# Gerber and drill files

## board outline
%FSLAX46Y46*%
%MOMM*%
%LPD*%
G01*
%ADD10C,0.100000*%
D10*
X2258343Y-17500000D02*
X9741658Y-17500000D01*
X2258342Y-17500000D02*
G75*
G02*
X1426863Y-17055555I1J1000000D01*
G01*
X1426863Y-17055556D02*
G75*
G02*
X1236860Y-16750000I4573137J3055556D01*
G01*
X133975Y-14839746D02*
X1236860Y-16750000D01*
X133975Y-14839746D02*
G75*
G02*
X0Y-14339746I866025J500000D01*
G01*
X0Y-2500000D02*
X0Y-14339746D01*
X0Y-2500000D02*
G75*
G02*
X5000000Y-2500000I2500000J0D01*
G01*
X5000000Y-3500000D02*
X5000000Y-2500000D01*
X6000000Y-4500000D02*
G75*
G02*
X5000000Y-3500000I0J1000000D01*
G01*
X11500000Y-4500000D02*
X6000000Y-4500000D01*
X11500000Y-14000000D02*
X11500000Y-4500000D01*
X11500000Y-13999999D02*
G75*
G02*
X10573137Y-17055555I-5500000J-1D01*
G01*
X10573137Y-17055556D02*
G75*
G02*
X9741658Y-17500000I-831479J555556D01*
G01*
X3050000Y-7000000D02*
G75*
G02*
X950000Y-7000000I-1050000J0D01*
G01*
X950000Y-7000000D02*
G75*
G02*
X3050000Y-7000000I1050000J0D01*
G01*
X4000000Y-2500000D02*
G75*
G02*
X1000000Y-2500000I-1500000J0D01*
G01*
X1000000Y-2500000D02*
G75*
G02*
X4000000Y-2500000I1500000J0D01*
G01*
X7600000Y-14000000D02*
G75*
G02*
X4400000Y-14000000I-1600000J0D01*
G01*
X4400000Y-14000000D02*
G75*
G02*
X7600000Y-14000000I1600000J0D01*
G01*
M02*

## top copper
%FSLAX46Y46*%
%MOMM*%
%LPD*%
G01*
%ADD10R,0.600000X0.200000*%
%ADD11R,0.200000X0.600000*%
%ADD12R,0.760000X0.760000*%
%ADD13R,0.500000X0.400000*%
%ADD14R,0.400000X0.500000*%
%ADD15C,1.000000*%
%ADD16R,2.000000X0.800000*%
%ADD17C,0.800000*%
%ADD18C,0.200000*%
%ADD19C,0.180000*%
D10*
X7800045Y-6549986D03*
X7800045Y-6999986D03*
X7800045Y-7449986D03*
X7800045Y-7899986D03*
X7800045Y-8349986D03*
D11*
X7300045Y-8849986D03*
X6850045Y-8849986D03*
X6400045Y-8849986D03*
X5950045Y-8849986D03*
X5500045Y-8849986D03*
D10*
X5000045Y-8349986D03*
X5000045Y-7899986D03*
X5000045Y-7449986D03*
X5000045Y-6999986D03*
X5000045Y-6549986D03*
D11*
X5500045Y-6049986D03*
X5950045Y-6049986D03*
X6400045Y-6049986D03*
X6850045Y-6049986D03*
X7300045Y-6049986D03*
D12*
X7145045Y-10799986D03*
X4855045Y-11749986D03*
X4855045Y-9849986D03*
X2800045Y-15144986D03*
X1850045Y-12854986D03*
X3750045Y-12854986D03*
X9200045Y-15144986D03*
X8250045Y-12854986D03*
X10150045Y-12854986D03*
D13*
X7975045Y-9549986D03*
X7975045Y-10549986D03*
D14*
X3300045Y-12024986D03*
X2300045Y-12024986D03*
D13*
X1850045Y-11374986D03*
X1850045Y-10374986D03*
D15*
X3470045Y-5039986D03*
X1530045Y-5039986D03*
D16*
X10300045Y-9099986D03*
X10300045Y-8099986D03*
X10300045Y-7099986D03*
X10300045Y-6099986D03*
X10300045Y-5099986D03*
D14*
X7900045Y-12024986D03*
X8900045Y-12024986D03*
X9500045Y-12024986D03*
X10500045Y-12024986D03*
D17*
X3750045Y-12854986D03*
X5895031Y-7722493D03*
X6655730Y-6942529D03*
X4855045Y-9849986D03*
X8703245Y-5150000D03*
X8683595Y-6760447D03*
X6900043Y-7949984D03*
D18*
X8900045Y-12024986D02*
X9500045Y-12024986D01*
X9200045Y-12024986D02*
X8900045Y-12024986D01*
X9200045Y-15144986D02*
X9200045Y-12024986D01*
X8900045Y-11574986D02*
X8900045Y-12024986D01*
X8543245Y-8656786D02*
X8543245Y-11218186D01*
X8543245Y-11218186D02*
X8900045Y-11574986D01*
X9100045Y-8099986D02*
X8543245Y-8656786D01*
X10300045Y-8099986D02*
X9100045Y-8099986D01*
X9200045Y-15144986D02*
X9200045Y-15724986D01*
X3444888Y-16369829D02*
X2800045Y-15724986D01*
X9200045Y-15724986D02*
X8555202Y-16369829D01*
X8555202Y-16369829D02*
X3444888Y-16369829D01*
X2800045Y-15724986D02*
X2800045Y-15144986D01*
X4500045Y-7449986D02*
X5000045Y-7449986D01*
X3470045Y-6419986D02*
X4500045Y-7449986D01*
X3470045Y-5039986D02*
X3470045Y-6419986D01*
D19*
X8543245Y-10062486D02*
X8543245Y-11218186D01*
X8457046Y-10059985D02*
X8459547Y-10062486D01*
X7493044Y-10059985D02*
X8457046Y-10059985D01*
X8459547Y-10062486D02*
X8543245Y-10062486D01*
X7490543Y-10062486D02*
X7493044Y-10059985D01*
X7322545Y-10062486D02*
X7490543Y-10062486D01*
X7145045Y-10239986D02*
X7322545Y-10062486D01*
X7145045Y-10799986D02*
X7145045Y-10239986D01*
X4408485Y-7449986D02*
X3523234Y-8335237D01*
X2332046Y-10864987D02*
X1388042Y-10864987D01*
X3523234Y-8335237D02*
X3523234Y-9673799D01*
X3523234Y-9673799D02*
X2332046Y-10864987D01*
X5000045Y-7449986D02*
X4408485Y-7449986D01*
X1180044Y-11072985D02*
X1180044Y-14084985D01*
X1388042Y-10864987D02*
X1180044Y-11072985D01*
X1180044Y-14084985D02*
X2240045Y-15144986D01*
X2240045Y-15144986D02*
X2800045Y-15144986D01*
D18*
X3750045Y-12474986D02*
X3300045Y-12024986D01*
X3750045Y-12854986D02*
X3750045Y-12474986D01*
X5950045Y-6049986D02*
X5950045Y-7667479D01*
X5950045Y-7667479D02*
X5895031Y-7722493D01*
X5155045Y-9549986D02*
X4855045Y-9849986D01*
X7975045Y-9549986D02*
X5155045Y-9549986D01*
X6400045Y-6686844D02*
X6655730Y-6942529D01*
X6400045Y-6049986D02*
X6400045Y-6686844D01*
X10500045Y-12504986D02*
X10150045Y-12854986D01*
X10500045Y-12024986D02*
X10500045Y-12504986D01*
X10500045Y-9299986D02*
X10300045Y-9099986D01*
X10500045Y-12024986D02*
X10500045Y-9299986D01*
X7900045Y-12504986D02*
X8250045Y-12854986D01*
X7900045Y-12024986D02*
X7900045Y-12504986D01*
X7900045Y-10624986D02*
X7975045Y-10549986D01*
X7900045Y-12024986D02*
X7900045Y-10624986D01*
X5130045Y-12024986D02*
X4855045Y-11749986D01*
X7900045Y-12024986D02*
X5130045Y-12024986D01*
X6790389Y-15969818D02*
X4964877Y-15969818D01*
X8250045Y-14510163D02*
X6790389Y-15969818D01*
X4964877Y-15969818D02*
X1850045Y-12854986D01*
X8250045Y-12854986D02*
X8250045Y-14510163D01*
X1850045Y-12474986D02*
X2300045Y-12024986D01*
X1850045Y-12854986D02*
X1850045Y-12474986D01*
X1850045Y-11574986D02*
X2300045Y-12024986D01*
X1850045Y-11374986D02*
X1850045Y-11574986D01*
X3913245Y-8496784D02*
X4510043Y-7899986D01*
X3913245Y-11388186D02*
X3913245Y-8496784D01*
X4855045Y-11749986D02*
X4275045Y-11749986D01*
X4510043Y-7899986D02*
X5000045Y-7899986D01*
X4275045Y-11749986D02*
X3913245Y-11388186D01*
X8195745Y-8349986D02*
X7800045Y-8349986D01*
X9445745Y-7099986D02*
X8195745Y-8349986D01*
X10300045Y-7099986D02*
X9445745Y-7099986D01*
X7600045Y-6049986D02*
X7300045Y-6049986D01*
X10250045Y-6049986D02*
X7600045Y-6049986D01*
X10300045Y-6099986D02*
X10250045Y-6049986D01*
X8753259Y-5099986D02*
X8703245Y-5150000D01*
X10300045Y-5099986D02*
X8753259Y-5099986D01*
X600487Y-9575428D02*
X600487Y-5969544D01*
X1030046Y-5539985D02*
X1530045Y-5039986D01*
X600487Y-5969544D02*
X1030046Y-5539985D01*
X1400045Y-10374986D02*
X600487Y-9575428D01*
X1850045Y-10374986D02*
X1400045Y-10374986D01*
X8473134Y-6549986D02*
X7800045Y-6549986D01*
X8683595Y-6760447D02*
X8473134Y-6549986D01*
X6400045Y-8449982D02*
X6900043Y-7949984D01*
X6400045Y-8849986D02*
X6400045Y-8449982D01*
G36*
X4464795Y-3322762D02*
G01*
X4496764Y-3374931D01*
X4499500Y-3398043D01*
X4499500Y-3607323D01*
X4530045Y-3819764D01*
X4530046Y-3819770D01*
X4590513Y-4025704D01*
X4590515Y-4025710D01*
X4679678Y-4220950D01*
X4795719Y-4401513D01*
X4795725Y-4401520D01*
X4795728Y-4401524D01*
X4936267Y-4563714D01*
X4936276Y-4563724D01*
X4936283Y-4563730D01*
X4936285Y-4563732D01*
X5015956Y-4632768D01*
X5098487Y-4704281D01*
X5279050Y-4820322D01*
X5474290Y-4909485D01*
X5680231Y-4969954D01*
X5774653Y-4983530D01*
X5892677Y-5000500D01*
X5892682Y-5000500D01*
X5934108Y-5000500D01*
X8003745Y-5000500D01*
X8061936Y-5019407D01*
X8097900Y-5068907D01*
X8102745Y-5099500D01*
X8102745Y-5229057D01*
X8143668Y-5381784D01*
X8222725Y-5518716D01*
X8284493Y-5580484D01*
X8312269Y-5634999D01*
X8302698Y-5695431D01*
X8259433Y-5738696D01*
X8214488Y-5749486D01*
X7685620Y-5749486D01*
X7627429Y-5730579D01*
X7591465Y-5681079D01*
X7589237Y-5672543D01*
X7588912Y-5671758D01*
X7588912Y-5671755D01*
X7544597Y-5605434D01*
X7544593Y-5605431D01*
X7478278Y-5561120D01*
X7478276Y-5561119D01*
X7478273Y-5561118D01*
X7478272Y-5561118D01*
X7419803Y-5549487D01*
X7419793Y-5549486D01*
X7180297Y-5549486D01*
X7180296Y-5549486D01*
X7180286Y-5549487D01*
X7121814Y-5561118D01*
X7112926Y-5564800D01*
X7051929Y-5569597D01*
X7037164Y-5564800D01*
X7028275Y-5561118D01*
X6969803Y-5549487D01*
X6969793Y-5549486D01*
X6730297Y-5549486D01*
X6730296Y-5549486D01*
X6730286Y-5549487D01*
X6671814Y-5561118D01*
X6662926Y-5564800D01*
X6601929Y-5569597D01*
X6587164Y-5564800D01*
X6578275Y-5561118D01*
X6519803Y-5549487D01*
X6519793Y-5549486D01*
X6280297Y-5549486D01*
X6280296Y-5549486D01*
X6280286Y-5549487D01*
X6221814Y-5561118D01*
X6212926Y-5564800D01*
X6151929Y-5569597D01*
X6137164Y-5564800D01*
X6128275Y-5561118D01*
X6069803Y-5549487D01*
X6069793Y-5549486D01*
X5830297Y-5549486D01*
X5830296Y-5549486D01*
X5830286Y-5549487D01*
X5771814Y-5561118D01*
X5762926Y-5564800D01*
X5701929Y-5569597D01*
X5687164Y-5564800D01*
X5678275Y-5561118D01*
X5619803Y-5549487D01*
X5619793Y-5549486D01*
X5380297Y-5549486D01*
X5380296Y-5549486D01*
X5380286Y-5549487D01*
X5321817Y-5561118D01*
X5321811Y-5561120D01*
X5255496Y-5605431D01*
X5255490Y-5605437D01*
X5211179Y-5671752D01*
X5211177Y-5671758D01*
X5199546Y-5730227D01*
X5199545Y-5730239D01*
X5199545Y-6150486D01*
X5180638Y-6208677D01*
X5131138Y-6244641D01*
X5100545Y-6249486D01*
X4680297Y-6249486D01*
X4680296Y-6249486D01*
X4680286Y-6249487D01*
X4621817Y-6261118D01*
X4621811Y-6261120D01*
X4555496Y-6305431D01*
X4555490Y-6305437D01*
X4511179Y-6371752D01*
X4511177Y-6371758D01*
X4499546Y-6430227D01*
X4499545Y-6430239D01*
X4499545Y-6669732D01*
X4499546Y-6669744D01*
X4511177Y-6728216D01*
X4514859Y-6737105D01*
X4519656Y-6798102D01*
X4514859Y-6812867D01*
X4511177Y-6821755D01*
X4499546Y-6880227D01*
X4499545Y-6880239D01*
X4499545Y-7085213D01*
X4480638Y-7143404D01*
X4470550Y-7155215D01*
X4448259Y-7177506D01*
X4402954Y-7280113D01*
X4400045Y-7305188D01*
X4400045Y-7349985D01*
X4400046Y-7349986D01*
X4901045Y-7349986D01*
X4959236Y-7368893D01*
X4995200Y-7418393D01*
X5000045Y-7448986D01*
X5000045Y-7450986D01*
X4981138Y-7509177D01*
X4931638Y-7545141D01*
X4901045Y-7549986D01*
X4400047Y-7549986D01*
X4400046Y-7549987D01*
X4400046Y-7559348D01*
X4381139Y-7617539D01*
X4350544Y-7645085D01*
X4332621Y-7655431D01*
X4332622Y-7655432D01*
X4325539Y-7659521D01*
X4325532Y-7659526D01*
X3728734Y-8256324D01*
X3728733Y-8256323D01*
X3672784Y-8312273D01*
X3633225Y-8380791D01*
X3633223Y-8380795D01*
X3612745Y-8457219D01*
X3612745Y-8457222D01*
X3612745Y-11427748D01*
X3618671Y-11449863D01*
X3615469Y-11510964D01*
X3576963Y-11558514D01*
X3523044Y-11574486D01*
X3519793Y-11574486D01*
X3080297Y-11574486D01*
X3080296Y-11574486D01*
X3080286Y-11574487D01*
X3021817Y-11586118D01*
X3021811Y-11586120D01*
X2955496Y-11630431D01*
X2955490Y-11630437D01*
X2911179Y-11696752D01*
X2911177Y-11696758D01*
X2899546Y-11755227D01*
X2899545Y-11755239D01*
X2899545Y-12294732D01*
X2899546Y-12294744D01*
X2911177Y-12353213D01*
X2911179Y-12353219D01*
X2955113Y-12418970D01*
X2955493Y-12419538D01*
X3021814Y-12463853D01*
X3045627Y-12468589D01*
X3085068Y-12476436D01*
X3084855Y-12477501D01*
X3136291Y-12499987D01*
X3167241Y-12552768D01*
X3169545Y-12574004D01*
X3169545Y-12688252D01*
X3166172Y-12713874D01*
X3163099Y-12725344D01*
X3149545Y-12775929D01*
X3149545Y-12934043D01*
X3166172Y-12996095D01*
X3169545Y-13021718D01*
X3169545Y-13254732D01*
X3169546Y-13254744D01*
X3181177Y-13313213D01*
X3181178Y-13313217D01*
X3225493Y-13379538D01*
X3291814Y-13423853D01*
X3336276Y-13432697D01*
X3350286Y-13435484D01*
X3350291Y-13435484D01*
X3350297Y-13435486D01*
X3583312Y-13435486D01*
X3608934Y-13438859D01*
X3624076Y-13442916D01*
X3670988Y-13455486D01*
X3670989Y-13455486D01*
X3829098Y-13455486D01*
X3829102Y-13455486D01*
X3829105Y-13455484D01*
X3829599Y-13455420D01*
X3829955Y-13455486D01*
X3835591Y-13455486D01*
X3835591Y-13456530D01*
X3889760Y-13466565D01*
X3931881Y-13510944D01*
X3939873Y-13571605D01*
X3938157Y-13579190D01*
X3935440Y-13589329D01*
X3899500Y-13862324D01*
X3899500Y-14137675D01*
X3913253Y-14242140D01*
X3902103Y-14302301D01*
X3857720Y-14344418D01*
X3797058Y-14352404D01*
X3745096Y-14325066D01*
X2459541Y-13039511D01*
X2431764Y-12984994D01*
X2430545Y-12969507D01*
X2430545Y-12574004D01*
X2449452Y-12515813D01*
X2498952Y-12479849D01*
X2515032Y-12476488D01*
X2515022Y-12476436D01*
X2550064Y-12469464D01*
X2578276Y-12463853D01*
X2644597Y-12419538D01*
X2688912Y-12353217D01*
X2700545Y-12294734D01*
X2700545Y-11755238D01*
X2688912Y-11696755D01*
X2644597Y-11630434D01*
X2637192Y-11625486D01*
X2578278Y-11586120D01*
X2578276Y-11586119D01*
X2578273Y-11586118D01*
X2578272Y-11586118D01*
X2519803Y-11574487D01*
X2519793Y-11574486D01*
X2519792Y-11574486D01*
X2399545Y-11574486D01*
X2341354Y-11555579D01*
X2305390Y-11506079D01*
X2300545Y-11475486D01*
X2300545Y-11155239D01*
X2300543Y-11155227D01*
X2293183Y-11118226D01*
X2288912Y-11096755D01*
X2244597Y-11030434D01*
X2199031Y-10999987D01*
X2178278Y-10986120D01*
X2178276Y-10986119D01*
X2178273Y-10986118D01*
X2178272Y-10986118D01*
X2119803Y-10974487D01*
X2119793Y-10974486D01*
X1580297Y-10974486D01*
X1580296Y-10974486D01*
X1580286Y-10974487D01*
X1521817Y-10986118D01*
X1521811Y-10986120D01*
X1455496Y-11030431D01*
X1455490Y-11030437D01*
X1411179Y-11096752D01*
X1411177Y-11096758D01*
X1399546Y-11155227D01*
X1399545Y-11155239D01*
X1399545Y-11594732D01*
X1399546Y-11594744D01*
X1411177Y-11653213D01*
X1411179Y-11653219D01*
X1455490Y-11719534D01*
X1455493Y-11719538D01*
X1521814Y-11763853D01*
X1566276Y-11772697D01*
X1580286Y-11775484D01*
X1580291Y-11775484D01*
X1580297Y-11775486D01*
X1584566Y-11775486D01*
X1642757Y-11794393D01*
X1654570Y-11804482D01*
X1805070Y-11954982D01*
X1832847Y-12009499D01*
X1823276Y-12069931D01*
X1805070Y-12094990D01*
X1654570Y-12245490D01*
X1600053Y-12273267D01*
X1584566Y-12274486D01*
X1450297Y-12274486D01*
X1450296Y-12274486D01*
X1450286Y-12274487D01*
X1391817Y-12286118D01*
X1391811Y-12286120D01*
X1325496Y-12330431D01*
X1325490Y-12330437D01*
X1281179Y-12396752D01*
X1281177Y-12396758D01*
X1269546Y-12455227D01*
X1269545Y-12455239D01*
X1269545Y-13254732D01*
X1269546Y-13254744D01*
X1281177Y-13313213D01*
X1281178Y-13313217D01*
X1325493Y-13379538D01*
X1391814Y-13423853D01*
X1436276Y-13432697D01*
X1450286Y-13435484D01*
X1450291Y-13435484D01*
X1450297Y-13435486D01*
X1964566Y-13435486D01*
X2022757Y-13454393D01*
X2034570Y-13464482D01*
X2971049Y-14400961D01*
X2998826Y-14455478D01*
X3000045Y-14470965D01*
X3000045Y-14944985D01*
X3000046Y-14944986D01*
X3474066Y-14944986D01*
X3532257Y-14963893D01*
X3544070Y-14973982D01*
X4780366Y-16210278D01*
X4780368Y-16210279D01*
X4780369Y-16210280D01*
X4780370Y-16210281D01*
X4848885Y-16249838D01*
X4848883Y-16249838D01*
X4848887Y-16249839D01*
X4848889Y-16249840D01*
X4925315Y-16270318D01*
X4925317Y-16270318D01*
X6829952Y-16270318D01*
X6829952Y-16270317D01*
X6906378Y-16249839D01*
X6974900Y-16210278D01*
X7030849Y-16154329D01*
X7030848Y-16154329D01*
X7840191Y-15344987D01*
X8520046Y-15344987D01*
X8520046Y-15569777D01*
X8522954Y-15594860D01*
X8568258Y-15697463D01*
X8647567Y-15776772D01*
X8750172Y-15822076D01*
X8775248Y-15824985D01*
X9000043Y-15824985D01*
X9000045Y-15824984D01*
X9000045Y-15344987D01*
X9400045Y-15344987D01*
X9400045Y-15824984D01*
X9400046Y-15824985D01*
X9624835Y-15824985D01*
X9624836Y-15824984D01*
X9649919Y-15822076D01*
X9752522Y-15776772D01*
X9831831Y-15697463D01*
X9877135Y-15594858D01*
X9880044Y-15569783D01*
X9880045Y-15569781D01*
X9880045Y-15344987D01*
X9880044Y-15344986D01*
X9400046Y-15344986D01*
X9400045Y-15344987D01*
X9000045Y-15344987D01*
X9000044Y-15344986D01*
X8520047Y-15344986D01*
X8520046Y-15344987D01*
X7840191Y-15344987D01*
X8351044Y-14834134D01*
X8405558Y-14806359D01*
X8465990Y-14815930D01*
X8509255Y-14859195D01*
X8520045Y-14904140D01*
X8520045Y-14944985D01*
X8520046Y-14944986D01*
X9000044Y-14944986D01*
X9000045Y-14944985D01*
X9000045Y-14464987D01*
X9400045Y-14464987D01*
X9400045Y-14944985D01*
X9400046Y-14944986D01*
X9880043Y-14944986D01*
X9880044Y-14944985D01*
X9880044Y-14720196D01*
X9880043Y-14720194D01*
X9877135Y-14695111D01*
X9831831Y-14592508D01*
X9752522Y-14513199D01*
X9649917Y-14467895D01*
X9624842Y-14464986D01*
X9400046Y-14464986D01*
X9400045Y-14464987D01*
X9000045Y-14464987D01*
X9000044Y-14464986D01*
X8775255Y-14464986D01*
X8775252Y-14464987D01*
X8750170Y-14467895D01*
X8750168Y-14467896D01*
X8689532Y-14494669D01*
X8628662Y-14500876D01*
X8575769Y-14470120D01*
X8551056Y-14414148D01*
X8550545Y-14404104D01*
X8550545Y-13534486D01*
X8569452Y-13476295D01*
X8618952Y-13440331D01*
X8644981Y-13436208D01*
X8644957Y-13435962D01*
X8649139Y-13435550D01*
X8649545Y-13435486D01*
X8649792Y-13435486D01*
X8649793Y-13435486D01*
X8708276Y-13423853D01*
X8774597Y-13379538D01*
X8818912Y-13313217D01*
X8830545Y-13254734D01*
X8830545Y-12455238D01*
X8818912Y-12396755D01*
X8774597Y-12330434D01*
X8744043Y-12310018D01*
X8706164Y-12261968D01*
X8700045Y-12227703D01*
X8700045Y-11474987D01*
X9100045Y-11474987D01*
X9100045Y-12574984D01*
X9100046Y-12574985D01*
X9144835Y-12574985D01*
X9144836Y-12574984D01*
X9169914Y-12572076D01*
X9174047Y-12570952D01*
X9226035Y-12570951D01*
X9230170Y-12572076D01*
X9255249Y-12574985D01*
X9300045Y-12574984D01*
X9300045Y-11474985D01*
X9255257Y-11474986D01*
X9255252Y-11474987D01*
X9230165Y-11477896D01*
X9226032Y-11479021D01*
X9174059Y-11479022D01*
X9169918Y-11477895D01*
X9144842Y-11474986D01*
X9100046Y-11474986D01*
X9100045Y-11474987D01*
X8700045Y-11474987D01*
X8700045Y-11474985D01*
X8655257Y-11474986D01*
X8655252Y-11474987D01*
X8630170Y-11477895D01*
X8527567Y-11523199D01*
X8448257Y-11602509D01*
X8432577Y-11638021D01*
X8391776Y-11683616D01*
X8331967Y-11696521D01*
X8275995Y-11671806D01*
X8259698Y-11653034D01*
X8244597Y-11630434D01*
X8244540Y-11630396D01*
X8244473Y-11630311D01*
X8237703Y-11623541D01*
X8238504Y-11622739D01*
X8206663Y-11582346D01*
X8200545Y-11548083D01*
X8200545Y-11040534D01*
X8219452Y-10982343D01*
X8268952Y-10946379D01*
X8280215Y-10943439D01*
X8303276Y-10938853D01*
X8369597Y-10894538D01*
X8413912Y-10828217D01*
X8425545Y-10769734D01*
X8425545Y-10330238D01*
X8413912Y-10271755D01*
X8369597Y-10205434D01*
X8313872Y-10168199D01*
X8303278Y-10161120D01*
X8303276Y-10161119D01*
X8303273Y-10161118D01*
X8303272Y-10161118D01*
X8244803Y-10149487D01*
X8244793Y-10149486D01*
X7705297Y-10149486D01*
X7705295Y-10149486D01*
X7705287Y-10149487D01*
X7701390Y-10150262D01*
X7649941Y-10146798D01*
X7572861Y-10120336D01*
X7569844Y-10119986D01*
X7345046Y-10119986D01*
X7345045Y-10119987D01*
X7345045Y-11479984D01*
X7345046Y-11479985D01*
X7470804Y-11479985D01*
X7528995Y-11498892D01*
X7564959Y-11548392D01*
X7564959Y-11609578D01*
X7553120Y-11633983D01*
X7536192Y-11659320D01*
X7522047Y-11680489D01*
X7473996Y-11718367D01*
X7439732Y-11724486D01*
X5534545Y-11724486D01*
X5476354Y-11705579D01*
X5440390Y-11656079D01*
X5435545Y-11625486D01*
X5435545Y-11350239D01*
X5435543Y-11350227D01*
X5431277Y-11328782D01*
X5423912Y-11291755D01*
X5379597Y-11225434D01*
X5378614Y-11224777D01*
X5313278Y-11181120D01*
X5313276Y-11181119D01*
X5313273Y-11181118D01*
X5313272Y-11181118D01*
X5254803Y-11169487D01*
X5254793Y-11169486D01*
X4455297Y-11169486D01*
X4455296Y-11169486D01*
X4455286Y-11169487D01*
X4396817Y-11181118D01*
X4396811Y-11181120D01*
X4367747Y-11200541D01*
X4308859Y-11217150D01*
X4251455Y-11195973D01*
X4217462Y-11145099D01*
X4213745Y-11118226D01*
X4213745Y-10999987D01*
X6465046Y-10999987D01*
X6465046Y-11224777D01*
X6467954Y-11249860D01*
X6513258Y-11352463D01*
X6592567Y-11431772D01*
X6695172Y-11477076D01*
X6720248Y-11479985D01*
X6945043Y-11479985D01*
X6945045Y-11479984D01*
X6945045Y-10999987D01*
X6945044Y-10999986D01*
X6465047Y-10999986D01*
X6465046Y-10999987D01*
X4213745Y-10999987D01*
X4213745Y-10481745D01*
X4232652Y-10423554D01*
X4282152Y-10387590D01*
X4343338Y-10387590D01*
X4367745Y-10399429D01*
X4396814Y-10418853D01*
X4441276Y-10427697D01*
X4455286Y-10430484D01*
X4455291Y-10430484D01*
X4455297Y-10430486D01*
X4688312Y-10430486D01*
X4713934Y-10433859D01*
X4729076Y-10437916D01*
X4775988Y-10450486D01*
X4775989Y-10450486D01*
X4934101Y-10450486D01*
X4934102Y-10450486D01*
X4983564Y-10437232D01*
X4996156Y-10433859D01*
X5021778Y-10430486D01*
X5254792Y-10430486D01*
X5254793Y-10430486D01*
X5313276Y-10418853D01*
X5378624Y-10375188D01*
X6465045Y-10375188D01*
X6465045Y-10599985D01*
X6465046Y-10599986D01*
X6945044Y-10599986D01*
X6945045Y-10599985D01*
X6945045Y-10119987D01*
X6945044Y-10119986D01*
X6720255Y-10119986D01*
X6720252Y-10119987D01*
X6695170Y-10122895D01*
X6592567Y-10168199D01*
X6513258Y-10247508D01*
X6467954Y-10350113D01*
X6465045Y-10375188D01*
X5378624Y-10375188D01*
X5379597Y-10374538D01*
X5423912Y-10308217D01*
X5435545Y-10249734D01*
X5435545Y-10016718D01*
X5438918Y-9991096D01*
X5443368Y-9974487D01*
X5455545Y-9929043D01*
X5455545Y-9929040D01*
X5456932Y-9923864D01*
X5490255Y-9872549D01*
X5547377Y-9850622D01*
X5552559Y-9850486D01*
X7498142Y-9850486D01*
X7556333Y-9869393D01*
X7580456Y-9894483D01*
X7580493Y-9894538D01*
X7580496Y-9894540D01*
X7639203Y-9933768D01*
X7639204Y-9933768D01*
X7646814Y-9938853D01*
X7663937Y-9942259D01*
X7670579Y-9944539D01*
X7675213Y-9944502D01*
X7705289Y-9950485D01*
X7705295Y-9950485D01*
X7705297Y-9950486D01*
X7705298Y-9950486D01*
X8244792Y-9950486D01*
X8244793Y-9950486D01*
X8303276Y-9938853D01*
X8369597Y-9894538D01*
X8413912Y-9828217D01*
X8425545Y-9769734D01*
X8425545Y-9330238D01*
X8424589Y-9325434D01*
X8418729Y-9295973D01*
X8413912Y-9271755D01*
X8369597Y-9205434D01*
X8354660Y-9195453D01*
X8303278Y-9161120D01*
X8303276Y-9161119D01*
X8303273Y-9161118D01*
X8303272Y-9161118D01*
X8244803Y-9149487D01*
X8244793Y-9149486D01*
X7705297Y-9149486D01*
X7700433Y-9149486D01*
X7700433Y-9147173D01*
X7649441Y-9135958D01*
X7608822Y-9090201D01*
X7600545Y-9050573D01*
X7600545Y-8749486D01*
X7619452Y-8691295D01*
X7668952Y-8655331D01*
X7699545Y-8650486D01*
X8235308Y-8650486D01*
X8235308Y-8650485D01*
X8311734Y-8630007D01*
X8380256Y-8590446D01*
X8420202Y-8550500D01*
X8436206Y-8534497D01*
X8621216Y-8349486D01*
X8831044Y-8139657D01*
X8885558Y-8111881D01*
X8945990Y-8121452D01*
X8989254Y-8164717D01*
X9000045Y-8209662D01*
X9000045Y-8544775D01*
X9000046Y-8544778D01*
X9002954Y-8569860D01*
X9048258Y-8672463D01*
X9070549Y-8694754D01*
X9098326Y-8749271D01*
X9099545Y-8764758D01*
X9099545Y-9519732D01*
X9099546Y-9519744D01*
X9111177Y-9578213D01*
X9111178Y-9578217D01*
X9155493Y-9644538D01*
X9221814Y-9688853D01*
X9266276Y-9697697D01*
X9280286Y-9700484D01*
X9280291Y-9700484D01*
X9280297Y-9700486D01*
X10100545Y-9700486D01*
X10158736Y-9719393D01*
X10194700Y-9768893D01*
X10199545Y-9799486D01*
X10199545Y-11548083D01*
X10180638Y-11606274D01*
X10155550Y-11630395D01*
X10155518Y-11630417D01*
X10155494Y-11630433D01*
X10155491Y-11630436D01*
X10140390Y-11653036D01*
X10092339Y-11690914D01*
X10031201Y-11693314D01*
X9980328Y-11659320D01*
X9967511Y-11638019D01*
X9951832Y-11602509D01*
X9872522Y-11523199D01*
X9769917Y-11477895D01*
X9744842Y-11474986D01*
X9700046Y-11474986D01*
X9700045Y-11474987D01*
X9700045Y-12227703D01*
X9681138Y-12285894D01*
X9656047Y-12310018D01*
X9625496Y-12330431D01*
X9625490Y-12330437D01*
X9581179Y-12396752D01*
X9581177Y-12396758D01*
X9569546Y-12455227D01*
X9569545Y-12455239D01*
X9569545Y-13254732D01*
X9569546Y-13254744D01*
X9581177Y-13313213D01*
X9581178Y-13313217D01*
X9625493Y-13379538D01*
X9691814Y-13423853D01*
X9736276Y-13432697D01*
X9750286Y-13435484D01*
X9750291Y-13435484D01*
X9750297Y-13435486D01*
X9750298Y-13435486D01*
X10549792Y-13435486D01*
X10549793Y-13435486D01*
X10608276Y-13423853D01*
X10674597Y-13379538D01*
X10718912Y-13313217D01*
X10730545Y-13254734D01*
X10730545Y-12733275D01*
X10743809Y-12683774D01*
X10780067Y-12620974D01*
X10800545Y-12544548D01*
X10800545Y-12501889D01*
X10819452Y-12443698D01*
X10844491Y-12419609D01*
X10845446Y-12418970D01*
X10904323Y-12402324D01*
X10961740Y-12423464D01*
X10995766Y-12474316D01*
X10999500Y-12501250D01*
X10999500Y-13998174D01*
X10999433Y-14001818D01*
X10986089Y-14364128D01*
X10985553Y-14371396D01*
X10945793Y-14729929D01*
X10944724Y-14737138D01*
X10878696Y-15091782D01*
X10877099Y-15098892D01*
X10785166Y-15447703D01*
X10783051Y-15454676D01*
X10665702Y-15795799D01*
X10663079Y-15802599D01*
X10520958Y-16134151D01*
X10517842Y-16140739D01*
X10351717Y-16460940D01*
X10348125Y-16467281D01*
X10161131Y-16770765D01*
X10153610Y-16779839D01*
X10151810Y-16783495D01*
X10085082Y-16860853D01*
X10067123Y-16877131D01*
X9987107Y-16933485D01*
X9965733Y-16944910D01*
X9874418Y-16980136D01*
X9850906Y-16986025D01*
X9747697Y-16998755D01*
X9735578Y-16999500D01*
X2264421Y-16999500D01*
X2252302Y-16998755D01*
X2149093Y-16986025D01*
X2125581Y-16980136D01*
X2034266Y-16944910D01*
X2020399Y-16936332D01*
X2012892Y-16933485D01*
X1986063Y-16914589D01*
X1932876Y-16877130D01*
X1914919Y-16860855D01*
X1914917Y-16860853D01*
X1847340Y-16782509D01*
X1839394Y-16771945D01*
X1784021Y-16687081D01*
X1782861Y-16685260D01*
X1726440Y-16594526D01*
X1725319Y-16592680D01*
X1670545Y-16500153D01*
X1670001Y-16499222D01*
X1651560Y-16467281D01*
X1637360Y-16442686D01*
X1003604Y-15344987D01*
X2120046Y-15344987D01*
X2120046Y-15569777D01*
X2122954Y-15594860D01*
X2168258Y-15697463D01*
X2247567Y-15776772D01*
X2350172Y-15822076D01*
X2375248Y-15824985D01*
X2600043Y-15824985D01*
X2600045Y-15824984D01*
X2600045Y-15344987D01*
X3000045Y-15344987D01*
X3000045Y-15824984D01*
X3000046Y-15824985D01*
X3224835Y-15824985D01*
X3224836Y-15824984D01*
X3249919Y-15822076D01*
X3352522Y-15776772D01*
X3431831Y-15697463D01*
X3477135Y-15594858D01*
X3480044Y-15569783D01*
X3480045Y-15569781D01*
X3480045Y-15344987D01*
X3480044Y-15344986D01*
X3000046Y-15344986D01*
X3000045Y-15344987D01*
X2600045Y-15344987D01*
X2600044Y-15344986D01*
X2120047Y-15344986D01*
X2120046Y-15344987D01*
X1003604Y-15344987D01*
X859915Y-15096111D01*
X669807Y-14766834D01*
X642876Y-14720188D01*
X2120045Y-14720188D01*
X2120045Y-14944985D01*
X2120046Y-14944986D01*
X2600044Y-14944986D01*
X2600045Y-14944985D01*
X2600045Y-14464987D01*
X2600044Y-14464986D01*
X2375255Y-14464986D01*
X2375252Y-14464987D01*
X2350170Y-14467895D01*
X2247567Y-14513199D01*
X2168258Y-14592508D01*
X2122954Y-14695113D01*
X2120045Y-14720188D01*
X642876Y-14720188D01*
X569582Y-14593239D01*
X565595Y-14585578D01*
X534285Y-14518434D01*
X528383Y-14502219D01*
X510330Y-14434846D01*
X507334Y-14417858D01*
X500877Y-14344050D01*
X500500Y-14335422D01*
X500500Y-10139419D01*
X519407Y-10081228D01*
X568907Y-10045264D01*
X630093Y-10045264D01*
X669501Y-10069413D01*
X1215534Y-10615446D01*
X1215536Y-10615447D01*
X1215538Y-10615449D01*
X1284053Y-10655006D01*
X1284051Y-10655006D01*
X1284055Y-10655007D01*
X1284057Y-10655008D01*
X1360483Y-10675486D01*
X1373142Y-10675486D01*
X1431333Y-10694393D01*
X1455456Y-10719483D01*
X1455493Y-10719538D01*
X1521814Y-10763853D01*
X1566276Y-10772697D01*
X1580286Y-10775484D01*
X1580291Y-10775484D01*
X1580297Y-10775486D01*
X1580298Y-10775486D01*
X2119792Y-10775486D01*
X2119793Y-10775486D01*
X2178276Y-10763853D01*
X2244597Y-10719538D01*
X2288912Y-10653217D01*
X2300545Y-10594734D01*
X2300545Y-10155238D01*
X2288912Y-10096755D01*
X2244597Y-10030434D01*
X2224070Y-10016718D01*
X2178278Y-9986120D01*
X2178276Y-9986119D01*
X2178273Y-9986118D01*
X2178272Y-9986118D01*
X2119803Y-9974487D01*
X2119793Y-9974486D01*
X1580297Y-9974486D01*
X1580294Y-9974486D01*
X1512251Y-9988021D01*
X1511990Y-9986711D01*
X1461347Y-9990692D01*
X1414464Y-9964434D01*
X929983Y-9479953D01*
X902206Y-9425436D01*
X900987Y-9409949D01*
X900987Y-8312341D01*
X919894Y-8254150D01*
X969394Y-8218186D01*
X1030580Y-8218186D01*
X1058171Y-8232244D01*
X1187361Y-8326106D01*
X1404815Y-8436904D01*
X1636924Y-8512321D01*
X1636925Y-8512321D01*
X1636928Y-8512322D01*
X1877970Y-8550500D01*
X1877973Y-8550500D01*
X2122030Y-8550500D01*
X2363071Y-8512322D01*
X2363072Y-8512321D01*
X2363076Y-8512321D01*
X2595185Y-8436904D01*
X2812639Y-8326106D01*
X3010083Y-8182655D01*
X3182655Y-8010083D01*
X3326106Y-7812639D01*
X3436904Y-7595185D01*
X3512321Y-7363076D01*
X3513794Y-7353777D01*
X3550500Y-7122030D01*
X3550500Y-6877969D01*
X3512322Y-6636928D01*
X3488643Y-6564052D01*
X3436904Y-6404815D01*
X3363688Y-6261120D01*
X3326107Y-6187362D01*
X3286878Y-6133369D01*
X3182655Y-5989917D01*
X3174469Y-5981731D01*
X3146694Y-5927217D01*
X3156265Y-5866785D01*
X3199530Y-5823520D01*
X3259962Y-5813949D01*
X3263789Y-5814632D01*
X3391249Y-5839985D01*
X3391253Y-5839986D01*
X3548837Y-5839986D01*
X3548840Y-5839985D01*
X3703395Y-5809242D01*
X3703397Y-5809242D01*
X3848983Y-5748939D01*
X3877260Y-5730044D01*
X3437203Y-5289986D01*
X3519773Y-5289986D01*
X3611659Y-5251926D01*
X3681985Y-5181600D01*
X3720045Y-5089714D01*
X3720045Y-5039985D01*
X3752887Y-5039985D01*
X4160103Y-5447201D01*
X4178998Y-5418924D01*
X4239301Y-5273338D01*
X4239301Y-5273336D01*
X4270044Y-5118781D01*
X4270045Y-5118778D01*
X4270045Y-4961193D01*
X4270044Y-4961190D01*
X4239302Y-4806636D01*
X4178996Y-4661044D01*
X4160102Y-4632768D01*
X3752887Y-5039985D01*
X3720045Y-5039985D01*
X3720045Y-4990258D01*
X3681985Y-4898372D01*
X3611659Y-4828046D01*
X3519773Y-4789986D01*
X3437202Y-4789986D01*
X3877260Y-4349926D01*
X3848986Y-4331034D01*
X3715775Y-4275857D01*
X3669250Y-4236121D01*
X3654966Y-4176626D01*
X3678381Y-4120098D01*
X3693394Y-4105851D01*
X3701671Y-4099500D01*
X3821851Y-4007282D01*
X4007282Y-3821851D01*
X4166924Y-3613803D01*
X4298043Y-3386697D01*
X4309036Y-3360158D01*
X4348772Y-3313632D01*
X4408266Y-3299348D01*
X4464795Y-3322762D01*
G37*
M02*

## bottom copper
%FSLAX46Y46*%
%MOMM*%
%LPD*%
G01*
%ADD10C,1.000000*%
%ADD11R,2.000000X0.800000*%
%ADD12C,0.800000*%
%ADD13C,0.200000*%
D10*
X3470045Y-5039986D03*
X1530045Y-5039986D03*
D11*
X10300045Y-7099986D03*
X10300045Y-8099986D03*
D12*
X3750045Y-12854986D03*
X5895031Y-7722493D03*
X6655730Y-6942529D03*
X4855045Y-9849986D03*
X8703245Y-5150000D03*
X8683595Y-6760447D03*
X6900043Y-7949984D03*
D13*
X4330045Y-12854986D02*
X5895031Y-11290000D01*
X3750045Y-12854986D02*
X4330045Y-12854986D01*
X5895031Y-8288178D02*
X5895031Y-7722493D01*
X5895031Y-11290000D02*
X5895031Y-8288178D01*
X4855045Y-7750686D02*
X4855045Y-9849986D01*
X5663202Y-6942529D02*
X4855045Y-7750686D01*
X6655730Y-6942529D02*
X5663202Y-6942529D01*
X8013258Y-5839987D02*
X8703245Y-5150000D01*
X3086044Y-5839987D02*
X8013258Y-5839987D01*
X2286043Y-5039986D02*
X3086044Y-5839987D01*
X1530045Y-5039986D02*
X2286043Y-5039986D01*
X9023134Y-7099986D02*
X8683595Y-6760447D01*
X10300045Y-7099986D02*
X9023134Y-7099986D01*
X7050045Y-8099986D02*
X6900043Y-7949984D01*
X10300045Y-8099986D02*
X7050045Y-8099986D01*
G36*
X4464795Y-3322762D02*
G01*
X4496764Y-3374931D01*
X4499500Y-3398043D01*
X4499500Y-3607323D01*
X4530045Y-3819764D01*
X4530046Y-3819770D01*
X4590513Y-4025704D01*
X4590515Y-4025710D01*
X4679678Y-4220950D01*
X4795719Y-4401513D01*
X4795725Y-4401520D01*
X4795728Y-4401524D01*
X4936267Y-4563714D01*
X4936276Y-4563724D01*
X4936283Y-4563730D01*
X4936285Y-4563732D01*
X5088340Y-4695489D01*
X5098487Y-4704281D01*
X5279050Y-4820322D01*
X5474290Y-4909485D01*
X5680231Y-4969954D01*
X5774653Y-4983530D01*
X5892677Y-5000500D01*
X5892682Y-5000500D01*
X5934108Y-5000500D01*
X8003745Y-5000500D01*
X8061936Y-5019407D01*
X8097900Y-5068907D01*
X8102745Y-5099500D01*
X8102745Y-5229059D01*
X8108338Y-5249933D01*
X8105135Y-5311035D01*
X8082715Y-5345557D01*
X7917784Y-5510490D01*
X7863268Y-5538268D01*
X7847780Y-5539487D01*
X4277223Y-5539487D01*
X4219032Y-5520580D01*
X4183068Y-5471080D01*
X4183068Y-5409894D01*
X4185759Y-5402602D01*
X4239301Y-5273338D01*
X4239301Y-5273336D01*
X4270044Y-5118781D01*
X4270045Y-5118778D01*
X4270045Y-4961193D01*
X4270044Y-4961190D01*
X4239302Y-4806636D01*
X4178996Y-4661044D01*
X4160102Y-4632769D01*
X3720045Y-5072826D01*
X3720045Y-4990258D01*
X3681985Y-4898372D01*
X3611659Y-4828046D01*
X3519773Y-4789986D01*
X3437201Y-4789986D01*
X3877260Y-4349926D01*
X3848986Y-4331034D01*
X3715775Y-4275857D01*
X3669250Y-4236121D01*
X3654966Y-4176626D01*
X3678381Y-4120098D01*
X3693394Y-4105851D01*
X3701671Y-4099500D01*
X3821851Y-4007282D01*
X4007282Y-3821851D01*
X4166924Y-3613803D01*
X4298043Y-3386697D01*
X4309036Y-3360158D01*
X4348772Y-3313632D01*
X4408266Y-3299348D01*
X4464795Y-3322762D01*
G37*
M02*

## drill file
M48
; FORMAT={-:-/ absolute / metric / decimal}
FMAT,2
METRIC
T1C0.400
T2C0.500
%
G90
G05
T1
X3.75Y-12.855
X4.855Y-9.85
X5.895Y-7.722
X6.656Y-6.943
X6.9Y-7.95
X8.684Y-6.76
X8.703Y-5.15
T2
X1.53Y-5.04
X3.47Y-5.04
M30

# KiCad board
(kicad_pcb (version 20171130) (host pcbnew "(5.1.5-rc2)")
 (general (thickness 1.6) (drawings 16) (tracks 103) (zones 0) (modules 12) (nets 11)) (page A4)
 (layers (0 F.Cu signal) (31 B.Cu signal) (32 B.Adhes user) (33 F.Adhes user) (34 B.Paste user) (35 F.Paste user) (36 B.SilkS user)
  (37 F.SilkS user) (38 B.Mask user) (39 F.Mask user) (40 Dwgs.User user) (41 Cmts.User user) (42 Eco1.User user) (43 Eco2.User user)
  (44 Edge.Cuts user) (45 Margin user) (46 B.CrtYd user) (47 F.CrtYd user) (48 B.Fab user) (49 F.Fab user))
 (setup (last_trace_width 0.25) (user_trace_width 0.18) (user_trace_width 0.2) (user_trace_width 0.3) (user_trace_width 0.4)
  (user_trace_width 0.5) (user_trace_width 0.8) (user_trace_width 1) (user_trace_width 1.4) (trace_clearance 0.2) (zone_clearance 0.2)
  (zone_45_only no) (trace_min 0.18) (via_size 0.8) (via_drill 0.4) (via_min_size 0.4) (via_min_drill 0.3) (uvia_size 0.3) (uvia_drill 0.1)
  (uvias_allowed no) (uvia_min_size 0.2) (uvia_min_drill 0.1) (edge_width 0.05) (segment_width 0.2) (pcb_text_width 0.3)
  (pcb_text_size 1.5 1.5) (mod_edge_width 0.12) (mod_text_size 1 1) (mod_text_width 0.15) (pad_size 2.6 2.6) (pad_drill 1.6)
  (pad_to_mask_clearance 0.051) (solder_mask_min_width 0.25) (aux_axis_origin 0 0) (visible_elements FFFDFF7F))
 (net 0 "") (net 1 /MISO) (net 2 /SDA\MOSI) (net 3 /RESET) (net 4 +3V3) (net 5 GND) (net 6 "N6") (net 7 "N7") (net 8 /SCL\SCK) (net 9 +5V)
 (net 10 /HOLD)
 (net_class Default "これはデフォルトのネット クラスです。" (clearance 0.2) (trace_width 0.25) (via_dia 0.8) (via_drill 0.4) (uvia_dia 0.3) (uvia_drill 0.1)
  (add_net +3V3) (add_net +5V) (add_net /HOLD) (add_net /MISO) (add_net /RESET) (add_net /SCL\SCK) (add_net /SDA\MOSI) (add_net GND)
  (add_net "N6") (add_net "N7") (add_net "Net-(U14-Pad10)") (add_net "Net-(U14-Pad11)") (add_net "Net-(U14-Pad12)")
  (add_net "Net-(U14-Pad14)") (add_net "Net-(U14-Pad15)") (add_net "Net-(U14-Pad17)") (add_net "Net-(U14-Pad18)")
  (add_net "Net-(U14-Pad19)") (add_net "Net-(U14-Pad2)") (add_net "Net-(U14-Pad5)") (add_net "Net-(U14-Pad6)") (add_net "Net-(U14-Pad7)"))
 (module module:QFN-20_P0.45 (layer F.Cu) (at 6.400045 7.449986 270)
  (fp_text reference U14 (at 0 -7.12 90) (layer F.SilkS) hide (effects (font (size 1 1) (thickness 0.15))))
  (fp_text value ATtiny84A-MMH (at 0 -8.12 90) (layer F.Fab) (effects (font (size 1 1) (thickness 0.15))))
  (pad 20 smd rect (at -0.9 -1.4) (size 0.6 0.2) (layers F.Cu F.Paste F.Mask) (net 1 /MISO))
  (pad 19 smd rect (at -0.45 -1.4) (size 0.6 0.2) (layers F.Cu F.Paste F.Mask))
  (pad 18 smd rect (at 0 -1.4) (size 0.6 0.2) (layers F.Cu F.Paste F.Mask))
  (pad 17 smd rect (at 0.45 -1.4) (size 0.6 0.2) (layers F.Cu F.Paste F.Mask))
  (pad 16 smd rect (at 0.9 -1.4) (size 0.6 0.2) (layers F.Cu F.Paste F.Mask) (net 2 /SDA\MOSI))
  (pad 15 smd rect (at 1.4 -0.9 270) (size 0.6 0.2) (layers F.Cu F.Paste F.Mask))
  (pad 14 smd rect (at 1.4 -0.45 270) (size 0.6 0.2) (layers F.Cu F.Paste F.Mask))
  (pad 13 smd rect (at 1.4 0 270) (size 0.6 0.2) (layers F.Cu F.Paste F.Mask) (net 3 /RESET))
  (pad 12 smd rect (at 1.4 0.45 270) (size 0.6 0.2) (layers F.Cu F.Paste F.Mask))
  (pad 11 smd rect (at 1.4 0.9 270) (size 0.6 0.2) (layers F.Cu F.Paste F.Mask))
  (pad 10 smd rect (at 0.9 1.4) (size 0.6 0.2) (layers F.Cu F.Paste F.Mask))
  (pad 9 smd rect (at 0.45 1.4) (size 0.6 0.2) (layers F.Cu F.Paste F.Mask) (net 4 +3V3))
  (pad 8 smd rect (at 0 1.4) (size 0.6 0.2) (layers F.Cu F.Paste F.Mask) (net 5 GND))
  (pad 7 smd rect (at -0.45 1.4) (size 0.6 0.2) (layers F.Cu F.Paste F.Mask))
  (pad 6 smd rect (at -0.9 1.4) (size 0.6 0.2) (layers F.Cu F.Paste F.Mask))
  (pad 5 smd rect (at -1.4 0.9 270) (size 0.6 0.2) (layers F.Cu F.Paste F.Mask))
  (pad 4 smd rect (at -1.4 0.45 270) (size 0.6 0.2) (layers F.Cu F.Paste F.Mask) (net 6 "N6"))
  (pad 3 smd rect (at -1.4 0 270) (size 0.6 0.2) (layers F.Cu F.Paste F.Mask) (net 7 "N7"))
  (pad 2 smd rect (at -1.4 -0.45 270) (size 0.6 0.2) (layers F.Cu F.Paste F.Mask))
  (pad 1 smd rect (at -1.4 -0.9 270) (size 0.6 0.2) (layers F.Cu F.Paste F.Mask) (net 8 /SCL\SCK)))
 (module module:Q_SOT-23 (layer F.Cu) (at 6.000045 10.799986 270)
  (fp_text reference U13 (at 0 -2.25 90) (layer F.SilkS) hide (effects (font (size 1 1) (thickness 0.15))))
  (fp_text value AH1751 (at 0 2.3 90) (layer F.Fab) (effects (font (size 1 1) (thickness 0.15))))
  (pad 3 smd rect (at 0 -1.145 270) (size 0.76 0.76) (layers F.Cu F.Paste F.Mask) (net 5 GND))
  (pad 2 smd rect (at 0.95 1.145 270) (size 0.76 0.76) (layers F.Cu F.Paste F.Mask) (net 4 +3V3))
  (pad 1 smd rect (at -0.95 1.145 270) (size 0.76 0.76) (layers F.Cu F.Paste F.Mask) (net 7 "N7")))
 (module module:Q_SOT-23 (layer F.Cu) (at 2.800045 13.999986 180)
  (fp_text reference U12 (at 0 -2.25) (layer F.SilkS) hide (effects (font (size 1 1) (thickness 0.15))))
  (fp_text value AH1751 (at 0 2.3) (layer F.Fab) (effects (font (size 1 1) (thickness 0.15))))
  (pad 3 smd rect (at 0 -1.145 180) (size 0.76 0.76) (layers F.Cu F.Paste F.Mask) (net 5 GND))
  (pad 2 smd rect (at 0.95 1.145 180) (size 0.76 0.76) (layers F.Cu F.Paste F.Mask) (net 4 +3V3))
  (pad 1 smd rect (at -0.95 1.145 180) (size 0.76 0.76) (layers F.Cu F.Paste F.Mask) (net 6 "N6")))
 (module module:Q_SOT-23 (layer F.Cu) (at 9.200045 13.999986 180)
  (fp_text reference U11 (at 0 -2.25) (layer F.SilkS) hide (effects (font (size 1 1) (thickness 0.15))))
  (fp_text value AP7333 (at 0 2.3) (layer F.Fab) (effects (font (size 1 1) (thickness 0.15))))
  (pad 3 smd rect (at 0 -1.145 180) (size 0.76 0.76) (layers F.Cu F.Paste F.Mask) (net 5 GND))
  (pad 2 smd rect (at 0.95 1.145 180) (size 0.76 0.76) (layers F.Cu F.Paste F.Mask) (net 4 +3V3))
  (pad 1 smd rect (at -0.95 1.145 180) (size 0.76 0.76) (layers F.Cu F.Paste F.Mask) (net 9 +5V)))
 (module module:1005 (layer F.Cu) (at 7.975045 10.049986 90)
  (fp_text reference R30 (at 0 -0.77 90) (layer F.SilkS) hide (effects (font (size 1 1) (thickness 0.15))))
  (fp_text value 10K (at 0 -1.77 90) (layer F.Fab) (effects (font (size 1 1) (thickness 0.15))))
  (pad 2 smd rect (at 0.5 0 90) (size 0.4 0.5) (layers F.Cu F.Paste F.Mask) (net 7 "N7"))
  (pad 1 smd rect (at -0.5 0 90) (size 0.4 0.5) (layers F.Cu F.Paste F.Mask) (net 4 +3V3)))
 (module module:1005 (layer F.Cu) (at 2.800045 12.024986)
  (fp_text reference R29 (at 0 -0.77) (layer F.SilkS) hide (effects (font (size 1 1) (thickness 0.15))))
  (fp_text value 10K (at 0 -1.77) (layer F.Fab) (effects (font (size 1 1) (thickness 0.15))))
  (pad 2 smd rect (at 0.5 0) (size 0.4 0.5) (layers F.Cu F.Paste F.Mask) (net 6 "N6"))
  (pad 1 smd rect (at -0.5 0) (size 0.4 0.5) (layers F.Cu F.Paste F.Mask) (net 4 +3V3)))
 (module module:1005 (layer F.Cu) (at 1.850045 10.874986 270)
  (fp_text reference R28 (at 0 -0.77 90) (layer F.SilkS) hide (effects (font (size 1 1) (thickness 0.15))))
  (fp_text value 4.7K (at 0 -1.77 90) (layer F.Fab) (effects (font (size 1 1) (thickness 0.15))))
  (pad 2 smd rect (at 0.5 0 270) (size 0.4 0.5) (layers F.Cu F.Paste F.Mask) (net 4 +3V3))
  (pad 1 smd rect (at -0.5 0 270) (size 0.4 0.5) (layers F.Cu F.Paste F.Mask) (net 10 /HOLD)))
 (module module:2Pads (layer F.Cu) (at 2.500045 5.039986)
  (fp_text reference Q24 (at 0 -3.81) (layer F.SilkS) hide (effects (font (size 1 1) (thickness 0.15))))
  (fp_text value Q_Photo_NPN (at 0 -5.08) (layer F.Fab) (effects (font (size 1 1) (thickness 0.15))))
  (pad 2 thru_hole circle (at 0.97 0) (size 1 1) (drill 0.5) (layers *.Cu *.Mask) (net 5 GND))
  (pad 1 thru_hole circle (at -0.97 0) (size 1 1) (drill 0.5) (layers *.Cu *.Mask) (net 10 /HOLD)))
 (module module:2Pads (layer B.Cu) (at 10.300045 7.599986 90)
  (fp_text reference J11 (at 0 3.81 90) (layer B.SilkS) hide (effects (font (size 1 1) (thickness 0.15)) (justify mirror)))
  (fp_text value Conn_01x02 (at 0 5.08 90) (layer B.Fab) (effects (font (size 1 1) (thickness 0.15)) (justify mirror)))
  (pad 2 smd rect (at 0.5 0 90) (size 0.8 2) (layers B.Cu B.Paste B.Mask) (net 1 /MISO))
  (pad 1 smd rect (at -0.5 0 90) (size 0.8 2) (layers B.Cu B.Paste B.Mask) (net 3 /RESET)))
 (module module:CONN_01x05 (layer F.Cu) (at 10.300045 7.099986 270)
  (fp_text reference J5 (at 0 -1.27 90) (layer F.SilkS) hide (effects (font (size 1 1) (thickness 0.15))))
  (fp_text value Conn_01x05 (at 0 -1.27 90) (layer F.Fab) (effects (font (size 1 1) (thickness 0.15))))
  (pad 5 smd rect (at 2 0 270) (size 0.8 2) (layers F.Cu F.Paste F.Mask) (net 9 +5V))
  (pad 4 smd rect (at 1 0 270) (size 0.8 2) (layers F.Cu F.Paste F.Mask) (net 5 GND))
  (pad 3 smd rect (at 0 0 270) (size 0.8 2) (layers F.Cu F.Paste F.Mask) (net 2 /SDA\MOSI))
  (pad 2 smd rect (at -1 0 270) (size 0.8 2) (layers F.Cu F.Paste F.Mask) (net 8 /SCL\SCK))
  (pad 1 smd rect (at -2 0 270) (size 0.8 2) (layers F.Cu F.Paste F.Mask) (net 10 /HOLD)))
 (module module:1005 (layer F.Cu) (at 8.400045 12.024986 180)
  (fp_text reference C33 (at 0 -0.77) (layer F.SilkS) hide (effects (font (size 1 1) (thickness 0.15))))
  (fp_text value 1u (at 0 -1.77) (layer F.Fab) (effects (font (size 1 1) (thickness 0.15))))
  (pad 2 smd rect (at 0.5 0 180) (size 0.4 0.5) (layers F.Cu F.Paste F.Mask) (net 4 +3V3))
  (pad 1 smd rect (at -0.5 0 180) (size 0.4 0.5) (layers F.Cu F.Paste F.Mask) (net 5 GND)))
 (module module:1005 (layer F.Cu) (at 10.000045 12.024986 180)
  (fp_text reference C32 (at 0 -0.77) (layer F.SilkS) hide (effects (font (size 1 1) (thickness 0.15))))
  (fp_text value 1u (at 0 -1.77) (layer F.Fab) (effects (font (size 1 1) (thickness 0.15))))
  (pad 2 smd rect (at 0.5 0 180) (size 0.4 0.5) (layers F.Cu F.Paste F.Mask) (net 5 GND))
  (pad 1 smd rect (at -0.5 0 180) (size 0.4 0.5) (layers F.Cu F.Paste F.Mask) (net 9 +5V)))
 (gr_line (start 2.258343 17.5) (end 9.741658 17.5) (layer Edge.Cuts) (width 0.1))
 (gr_arc (start 2.258343 16.5) (end 1.426863 17.055555) (angle -56.2510114) (layer Edge.Cuts) (width 0.1))
 (gr_arc (start 6 14) (end 1.23686 16.75) (angle -3.748988596) (layer Edge.Cuts) (width 0.1))
 (gr_line (start 0.133975 14.839746) (end 1.23686 16.75) (layer Edge.Cuts) (width 0.1))
 (gr_arc (start 1 14.339746) (end 0 14.339746) (angle -30) (layer Edge.Cuts) (width 0.1))
 (gr_line (start 0 2.5) (end 0 14.339746) (layer Edge.Cuts) (width 0.1))
 (gr_arc (start 2.5 2.5) (end 5 2.5) (angle -180) (layer Edge.Cuts) (width 0.1))
 (gr_line (start 5 3.5) (end 5 2.5) (layer Edge.Cuts) (width 0.1))
 (gr_arc (start 6 3.5) (end 5 3.5) (angle -90) (layer Edge.Cuts) (width 0.1))
 (gr_line (start 11.5 4.5) (end 6 4.5) (layer Edge.Cuts) (width 0.1))
 (gr_line (start 11.5 14) (end 11.5 4.5) (layer Edge.Cuts) (width 0.1))
 (gr_arc (start 6 14) (end 10.573137 17.055555) (angle -33.7489886) (layer Edge.Cuts) (width 0.1))
 (gr_arc (start 9.741658 16.5) (end 9.741658 17.5) (angle -56.2510114) (layer Edge.Cuts) (width 0.1))
 (gr_circle (center 2 7) (end 2 5.95) (layer Edge.Cuts) (width 0.1))
 (gr_circle (center 2.5 2.5) (end 2.5 1) (layer Edge.Cuts) (width 0.1))
 (gr_circle (center 6 14) (end 6 12.4) (layer Edge.Cuts) (width 0.1))
 (segment (start 8.900045 12.024986) (end 9.500045 12.024986) (width 0.2) (layer F.Cu) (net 5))
 (segment (start 9.200045 12.024986) (end 8.900045 12.024986) (width 0.2) (layer F.Cu) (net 5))
 (segment (start 9.200045 15.144986) (end 9.200045 12.024986) (width 0.2) (layer F.Cu) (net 5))
 (segment (start 8.900045 11.574986) (end 8.900045 12.024986) (width 0.2) (layer F.Cu) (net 5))
 (segment (start 8.543245 8.656786) (end 8.543245 11.218186) (width 0.2) (layer F.Cu) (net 5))
 (segment (start 8.543245 11.218186) (end 8.900045 11.574986) (width 0.2) (layer F.Cu) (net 5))
 (segment (start 9.100045 8.099986) (end 8.543245 8.656786) (width 0.2) (layer F.Cu) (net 5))
 (segment (start 10.300045 8.099986) (end 9.100045 8.099986) (width 0.2) (layer F.Cu) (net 5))
 (segment (start 9.200045 15.144986) (end 9.200045 15.724986) (width 0.2) (layer F.Cu) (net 5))
 (segment (start 3.444888 16.369829) (end 2.800045 15.724986) (width 0.2) (layer F.Cu) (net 5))
 (segment (start 9.200045 15.724986) (end 8.555202 16.369829) (width 0.2) (layer F.Cu) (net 5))
 (segment (start 8.555202 16.369829) (end 3.444888 16.369829) (width 0.2) (layer F.Cu) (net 5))
 (segment (start 2.800045 15.724986) (end 2.800045 15.144986) (width 0.2) (layer F.Cu) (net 5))
 (segment (start 4.500045 7.449986) (end 5.000045 7.449986) (width 0.2) (layer F.Cu) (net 5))
 (segment (start 3.470045 6.419986) (end 4.500045 7.449986) (width 0.2) (layer F.Cu) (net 5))
 (segment (start 3.470045 5.039986) (end 3.470045 6.419986) (width 0.2) (layer F.Cu) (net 5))
 (segment (start 8.543245 10.062486) (end 8.543245 11.218186) (width 0.18) (layer F.Cu) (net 5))
 (segment (start 8.457046 10.059985) (end 8.459547 10.062486) (width 0.18) (layer F.Cu) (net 5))
 (segment (start 7.493044 10.059985) (end 8.457046 10.059985) (width 0.18) (layer F.Cu) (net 5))
 (segment (start 8.459547 10.062486) (end 8.543245 10.062486) (width 0.18) (layer F.Cu) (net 5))
 (segment (start 7.490543 10.062486) (end 7.493044 10.059985) (width 0.18) (layer F.Cu) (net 5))
 (segment (start 7.322545 10.062486) (end 7.490543 10.062486) (width 0.18) (layer F.Cu) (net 5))
 (segment (start 7.145045 10.239986) (end 7.322545 10.062486) (width 0.18) (layer F.Cu) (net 5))
 (segment (start 7.145045 10.799986) (end 7.145045 10.239986) (width 0.18) (layer F.Cu) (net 5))
 (segment (start 4.408485 7.449986) (end 3.523234 8.335237) (width 0.18) (layer F.Cu) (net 5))
 (segment (start 2.332046 10.864987) (end 1.388042 10.864987) (width 0.18) (layer F.Cu) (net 5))
 (segment (start 3.523234 8.335237) (end 3.523234 9.673799) (width 0.18) (layer F.Cu) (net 5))
 (segment (start 3.523234 9.673799) (end 2.332046 10.864987) (width 0.18) (layer F.Cu) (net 5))
 (segment (start 5.000045 7.449986) (end 4.408485 7.449986) (width 0.18) (layer F.Cu) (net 5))
 (segment (start 1.180044 11.072985) (end 1.180044 14.084985) (width 0.18) (layer F.Cu) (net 5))
 (segment (start 1.388042 10.864987) (end 1.180044 11.072985) (width 0.18) (layer F.Cu) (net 5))
 (segment (start 1.180044 14.084985) (end 2.240045 15.144986) (width 0.18) (layer F.Cu) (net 5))
 (segment (start 2.240045 15.144986) (end 2.800045 15.144986) (width 0.18) (layer F.Cu) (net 5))
 (segment (start 3.750045 12.474986) (end 3.300045 12.024986) (width 0.2) (layer F.Cu) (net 6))
 (segment (start 3.750045 12.854986) (end 3.750045 12.474986) (width 0.2) (layer F.Cu) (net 6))
 (via (at 3.750045 12.854986) (size 0.8) (drill 0.4) (layers F.Cu B.Cu) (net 6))
 (segment (start 5.950045 6.049986) (end 5.950045 7.667479) (width 0.2) (layer F.Cu) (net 6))
 (via (at 5.895031 7.722493) (size 0.8) (drill 0.4) (layers F.Cu B.Cu) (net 6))
 (segment (start 5.950045 7.667479) (end 5.895031 7.722493) (width 0.2) (layer F.Cu) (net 6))
 (segment (start 4.330045 12.854986) (end 5.895031 11.29) (width 0.2) (layer B.Cu) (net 6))
 (segment (start 3.750045 12.854986) (end 4.330045 12.854986) (width 0.2) (layer B.Cu) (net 6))
 (segment (start 5.895031 8.288178) (end 5.895031 7.722493) (width 0.2) (layer B.Cu) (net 6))
 (segment (start 5.895031 11.29) (end 5.895031 8.288178) (width 0.2) (layer B.Cu) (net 6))
 (segment (start 5.155045 9.549986) (end 4.855045 9.849986) (width 0.2) (layer F.Cu) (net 7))
 (segment (start 7.975045 9.549986) (end 5.155045 9.549986) (width 0.2) (layer F.Cu) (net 7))
 (via (at 6.65573 6.942529) (size 0.8) (drill 0.4) (layers F.Cu B.Cu) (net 7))
 (segment (start 6.400045 6.686844) (end 6.65573 6.942529) (width 0.2) (layer F.Cu) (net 7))
 (segment (start 6.400045 6.049986) (end 6.400045 6.686844) (width 0.2) (layer F.Cu) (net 7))
 (via (at 4.855045 9.849986) (size 0.8) (drill 0.4) (layers F.Cu B.Cu) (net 7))
 (segment (start 4.855045 7.750686) (end 4.855045 9.849986) (width 0.2) (layer B.Cu) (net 7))
 (segment (start 5.663202 6.942529) (end 4.855045 7.750686) (width 0.2) (layer B.Cu) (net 7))
 (segment (start 6.65573 6.942529) (end 5.663202 6.942529) (width 0.2) (layer B.Cu) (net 7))
 (segment (start 10.500045 12.504986) (end 10.150045 12.854986) (width 0.2) (layer F.Cu) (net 9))
 (segment (start 10.500045 12.024986) (end 10.500045 12.504986) (width 0.2) (layer F.Cu) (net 9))
 (segment (start 10.500045 9.299986) (end 10.300045 9.099986) (width 0.2) (layer F.Cu) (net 9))
 (segment (start 10.500045 12.024986) (end 10.500045 9.299986) (width 0.2) (layer F.Cu) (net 9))
 (segment (start 7.900045 12.504986) (end 8.250045 12.854986) (width 0.2) (layer F.Cu) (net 4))
 (segment (start 7.900045 12.024986) (end 7.900045 12.504986) (width 0.2) (layer F.Cu) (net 4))
 (segment (start 7.900045 10.624986) (end 7.975045 10.549986) (width 0.2) (layer F.Cu) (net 4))
 (segment (start 7.900045 12.024986) (end 7.900045 10.624986) (width 0.2) (layer F.Cu) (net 4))
 (segment (start 5.130045 12.024986) (end 4.855045 11.749986) (width 0.2) (layer F.Cu) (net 4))
 (segment (start 7.900045 12.024986) (end 5.130045 12.024986) (width 0.2) (layer F.Cu) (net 4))
 (segment (start 6.790389 15.969818) (end 4.964877 15.969818) (width 0.2) (layer F.Cu) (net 4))
 (segment (start 8.250045 14.510163) (end 6.790389 15.969818) (width 0.2) (layer F.Cu) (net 4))
 (segment (start 4.964877 15.969818) (end 1.850045 12.854986) (width 0.2) (layer F.Cu) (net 4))
 (segment (start 8.250045 12.854986) (end 8.250045 14.510163) (width 0.2) (layer F.Cu) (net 4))
 (segment (start 1.850045 12.474986) (end 2.300045 12.024986) (width 0.2) (layer F.Cu) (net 4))
 (segment (start 1.850045 12.854986) (end 1.850045 12.474986) (width 0.2) (layer F.Cu) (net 4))
 (segment (start 1.850045 11.574986) (end 2.300045 12.024986) (width 0.2) (layer F.Cu) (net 4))
 (segment (start 1.850045 11.374986) (end 1.850045 11.574986) (width 0.2) (layer F.Cu) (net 4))
 (segment (start 3.913245 8.496784) (end 4.510043 7.899986) (width 0.2) (layer F.Cu) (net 4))
 (segment (start 3.913245 11.388186) (end 3.913245 8.496784) (width 0.2) (layer F.Cu) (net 4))
 (segment (start 4.855045 11.749986) (end 4.275045 11.749986) (width 0.2) (layer F.Cu) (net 4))
 (segment (start 4.510043 7.899986) (end 5.000045 7.899986) (width 0.2) (layer F.Cu) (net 4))
 (segment (start 4.275045 11.749986) (end 3.913245 11.388186) (width 0.2) (layer F.Cu) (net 4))
 (segment (start 8.195745 8.349986) (end 7.800045 8.349986) (width 0.2) (layer F.Cu) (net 2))
 (segment (start 9.445745 7.099986) (end 8.195745 8.349986) (width 0.2) (layer F.Cu) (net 2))
 (segment (start 10.300045 7.099986) (end 9.445745 7.099986) (width 0.2) (layer F.Cu) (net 2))
 (segment (start 7.600045 6.049986) (end 7.300045 6.049986) (width 0.2) (layer F.Cu) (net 8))
 (segment (start 10.250045 6.049986) (end 7.600045 6.049986) (width 0.2) (layer F.Cu) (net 8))
 (segment (start 10.300045 6.099986) (end 10.250045 6.049986) (width 0.2) (layer F.Cu) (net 8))
 (via (at 8.703245 5.15) (size 0.8) (drill 0.4) (layers F.Cu B.Cu) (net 10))
 (segment (start 8.013258 5.839987) (end 8.703245 5.15) (width 0.2) (layer B.Cu) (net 10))
 (segment (start 3.086044 5.839987) (end 8.013258 5.839987) (width 0.2) (layer B.Cu) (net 10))
 (segment (start 2.286043 5.039986) (end 3.086044 5.839987) (width 0.2) (layer B.Cu) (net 10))
 (segment (start 1.530045 5.039986) (end 2.286043 5.039986) (width 0.2) (layer B.Cu) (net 10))
 (segment (start 8.753259 5.099986) (end 8.703245 5.15) (width 0.2) (layer F.Cu) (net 10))
 (segment (start 10.300045 5.099986) (end 8.753259 5.099986) (width 0.2) (layer F.Cu) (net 10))
 (segment (start 0.600487 9.575428) (end 0.600487 5.969544) (width 0.2) (layer F.Cu) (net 10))
 (segment (start 1.030046 5.539985) (end 1.530045 5.039986) (width 0.2) (layer F.Cu) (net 10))
 (segment (start 0.600487 5.969544) (end 1.030046 5.539985) (width 0.2) (layer F.Cu) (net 10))
 (segment (start 1.400045 10.374986) (end 0.600487 9.575428) (width 0.2) (layer F.Cu) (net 10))
 (segment (start 1.850045 10.374986) (end 1.400045 10.374986) (width 0.2) (layer F.Cu) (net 10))
 (via (at 8.683595 6.760447) (size 0.8) (drill 0.4) (layers F.Cu B.Cu) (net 1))
 (segment (start 9.023134 7.099986) (end 8.683595 6.760447) (width 0.2) (layer B.Cu) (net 1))
 (segment (start 10.300045 7.099986) (end 9.023134 7.099986) (width 0.2) (layer B.Cu) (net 1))
 (segment (start 8.473134 6.549986) (end 7.800045 6.549986) (width 0.2) (layer F.Cu) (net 1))
 (segment (start 8.683595 6.760447) (end 8.473134 6.549986) (width 0.2) (layer F.Cu) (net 1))
 (segment (start 6.400045 8.449982) (end 6.900043 7.949984) (width 0.2) (layer F.Cu) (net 3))
 (via (at 6.900043 7.949984) (size 0.8) (drill 0.4) (layers F.Cu B.Cu) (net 3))
 (segment (start 6.400045 8.849986) (end 6.400045 8.449982) (width 0.2) (layer F.Cu) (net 3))
 (segment (start 7.050045 8.099986) (end 6.900043 7.949984) (width 0.2) (layer B.Cu) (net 3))
 (segment (start 10.300045 8.099986) (end 7.050045 8.099986) (width 0.2) (layer B.Cu) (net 3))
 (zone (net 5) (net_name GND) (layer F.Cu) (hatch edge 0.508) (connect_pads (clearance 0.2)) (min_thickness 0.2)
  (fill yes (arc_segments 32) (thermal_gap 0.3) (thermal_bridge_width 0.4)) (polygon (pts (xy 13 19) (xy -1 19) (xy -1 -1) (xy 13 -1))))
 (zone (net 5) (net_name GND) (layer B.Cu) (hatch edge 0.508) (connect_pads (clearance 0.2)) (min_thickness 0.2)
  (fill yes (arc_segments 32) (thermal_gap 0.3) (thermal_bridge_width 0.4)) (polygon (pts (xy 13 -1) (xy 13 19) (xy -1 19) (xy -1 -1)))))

